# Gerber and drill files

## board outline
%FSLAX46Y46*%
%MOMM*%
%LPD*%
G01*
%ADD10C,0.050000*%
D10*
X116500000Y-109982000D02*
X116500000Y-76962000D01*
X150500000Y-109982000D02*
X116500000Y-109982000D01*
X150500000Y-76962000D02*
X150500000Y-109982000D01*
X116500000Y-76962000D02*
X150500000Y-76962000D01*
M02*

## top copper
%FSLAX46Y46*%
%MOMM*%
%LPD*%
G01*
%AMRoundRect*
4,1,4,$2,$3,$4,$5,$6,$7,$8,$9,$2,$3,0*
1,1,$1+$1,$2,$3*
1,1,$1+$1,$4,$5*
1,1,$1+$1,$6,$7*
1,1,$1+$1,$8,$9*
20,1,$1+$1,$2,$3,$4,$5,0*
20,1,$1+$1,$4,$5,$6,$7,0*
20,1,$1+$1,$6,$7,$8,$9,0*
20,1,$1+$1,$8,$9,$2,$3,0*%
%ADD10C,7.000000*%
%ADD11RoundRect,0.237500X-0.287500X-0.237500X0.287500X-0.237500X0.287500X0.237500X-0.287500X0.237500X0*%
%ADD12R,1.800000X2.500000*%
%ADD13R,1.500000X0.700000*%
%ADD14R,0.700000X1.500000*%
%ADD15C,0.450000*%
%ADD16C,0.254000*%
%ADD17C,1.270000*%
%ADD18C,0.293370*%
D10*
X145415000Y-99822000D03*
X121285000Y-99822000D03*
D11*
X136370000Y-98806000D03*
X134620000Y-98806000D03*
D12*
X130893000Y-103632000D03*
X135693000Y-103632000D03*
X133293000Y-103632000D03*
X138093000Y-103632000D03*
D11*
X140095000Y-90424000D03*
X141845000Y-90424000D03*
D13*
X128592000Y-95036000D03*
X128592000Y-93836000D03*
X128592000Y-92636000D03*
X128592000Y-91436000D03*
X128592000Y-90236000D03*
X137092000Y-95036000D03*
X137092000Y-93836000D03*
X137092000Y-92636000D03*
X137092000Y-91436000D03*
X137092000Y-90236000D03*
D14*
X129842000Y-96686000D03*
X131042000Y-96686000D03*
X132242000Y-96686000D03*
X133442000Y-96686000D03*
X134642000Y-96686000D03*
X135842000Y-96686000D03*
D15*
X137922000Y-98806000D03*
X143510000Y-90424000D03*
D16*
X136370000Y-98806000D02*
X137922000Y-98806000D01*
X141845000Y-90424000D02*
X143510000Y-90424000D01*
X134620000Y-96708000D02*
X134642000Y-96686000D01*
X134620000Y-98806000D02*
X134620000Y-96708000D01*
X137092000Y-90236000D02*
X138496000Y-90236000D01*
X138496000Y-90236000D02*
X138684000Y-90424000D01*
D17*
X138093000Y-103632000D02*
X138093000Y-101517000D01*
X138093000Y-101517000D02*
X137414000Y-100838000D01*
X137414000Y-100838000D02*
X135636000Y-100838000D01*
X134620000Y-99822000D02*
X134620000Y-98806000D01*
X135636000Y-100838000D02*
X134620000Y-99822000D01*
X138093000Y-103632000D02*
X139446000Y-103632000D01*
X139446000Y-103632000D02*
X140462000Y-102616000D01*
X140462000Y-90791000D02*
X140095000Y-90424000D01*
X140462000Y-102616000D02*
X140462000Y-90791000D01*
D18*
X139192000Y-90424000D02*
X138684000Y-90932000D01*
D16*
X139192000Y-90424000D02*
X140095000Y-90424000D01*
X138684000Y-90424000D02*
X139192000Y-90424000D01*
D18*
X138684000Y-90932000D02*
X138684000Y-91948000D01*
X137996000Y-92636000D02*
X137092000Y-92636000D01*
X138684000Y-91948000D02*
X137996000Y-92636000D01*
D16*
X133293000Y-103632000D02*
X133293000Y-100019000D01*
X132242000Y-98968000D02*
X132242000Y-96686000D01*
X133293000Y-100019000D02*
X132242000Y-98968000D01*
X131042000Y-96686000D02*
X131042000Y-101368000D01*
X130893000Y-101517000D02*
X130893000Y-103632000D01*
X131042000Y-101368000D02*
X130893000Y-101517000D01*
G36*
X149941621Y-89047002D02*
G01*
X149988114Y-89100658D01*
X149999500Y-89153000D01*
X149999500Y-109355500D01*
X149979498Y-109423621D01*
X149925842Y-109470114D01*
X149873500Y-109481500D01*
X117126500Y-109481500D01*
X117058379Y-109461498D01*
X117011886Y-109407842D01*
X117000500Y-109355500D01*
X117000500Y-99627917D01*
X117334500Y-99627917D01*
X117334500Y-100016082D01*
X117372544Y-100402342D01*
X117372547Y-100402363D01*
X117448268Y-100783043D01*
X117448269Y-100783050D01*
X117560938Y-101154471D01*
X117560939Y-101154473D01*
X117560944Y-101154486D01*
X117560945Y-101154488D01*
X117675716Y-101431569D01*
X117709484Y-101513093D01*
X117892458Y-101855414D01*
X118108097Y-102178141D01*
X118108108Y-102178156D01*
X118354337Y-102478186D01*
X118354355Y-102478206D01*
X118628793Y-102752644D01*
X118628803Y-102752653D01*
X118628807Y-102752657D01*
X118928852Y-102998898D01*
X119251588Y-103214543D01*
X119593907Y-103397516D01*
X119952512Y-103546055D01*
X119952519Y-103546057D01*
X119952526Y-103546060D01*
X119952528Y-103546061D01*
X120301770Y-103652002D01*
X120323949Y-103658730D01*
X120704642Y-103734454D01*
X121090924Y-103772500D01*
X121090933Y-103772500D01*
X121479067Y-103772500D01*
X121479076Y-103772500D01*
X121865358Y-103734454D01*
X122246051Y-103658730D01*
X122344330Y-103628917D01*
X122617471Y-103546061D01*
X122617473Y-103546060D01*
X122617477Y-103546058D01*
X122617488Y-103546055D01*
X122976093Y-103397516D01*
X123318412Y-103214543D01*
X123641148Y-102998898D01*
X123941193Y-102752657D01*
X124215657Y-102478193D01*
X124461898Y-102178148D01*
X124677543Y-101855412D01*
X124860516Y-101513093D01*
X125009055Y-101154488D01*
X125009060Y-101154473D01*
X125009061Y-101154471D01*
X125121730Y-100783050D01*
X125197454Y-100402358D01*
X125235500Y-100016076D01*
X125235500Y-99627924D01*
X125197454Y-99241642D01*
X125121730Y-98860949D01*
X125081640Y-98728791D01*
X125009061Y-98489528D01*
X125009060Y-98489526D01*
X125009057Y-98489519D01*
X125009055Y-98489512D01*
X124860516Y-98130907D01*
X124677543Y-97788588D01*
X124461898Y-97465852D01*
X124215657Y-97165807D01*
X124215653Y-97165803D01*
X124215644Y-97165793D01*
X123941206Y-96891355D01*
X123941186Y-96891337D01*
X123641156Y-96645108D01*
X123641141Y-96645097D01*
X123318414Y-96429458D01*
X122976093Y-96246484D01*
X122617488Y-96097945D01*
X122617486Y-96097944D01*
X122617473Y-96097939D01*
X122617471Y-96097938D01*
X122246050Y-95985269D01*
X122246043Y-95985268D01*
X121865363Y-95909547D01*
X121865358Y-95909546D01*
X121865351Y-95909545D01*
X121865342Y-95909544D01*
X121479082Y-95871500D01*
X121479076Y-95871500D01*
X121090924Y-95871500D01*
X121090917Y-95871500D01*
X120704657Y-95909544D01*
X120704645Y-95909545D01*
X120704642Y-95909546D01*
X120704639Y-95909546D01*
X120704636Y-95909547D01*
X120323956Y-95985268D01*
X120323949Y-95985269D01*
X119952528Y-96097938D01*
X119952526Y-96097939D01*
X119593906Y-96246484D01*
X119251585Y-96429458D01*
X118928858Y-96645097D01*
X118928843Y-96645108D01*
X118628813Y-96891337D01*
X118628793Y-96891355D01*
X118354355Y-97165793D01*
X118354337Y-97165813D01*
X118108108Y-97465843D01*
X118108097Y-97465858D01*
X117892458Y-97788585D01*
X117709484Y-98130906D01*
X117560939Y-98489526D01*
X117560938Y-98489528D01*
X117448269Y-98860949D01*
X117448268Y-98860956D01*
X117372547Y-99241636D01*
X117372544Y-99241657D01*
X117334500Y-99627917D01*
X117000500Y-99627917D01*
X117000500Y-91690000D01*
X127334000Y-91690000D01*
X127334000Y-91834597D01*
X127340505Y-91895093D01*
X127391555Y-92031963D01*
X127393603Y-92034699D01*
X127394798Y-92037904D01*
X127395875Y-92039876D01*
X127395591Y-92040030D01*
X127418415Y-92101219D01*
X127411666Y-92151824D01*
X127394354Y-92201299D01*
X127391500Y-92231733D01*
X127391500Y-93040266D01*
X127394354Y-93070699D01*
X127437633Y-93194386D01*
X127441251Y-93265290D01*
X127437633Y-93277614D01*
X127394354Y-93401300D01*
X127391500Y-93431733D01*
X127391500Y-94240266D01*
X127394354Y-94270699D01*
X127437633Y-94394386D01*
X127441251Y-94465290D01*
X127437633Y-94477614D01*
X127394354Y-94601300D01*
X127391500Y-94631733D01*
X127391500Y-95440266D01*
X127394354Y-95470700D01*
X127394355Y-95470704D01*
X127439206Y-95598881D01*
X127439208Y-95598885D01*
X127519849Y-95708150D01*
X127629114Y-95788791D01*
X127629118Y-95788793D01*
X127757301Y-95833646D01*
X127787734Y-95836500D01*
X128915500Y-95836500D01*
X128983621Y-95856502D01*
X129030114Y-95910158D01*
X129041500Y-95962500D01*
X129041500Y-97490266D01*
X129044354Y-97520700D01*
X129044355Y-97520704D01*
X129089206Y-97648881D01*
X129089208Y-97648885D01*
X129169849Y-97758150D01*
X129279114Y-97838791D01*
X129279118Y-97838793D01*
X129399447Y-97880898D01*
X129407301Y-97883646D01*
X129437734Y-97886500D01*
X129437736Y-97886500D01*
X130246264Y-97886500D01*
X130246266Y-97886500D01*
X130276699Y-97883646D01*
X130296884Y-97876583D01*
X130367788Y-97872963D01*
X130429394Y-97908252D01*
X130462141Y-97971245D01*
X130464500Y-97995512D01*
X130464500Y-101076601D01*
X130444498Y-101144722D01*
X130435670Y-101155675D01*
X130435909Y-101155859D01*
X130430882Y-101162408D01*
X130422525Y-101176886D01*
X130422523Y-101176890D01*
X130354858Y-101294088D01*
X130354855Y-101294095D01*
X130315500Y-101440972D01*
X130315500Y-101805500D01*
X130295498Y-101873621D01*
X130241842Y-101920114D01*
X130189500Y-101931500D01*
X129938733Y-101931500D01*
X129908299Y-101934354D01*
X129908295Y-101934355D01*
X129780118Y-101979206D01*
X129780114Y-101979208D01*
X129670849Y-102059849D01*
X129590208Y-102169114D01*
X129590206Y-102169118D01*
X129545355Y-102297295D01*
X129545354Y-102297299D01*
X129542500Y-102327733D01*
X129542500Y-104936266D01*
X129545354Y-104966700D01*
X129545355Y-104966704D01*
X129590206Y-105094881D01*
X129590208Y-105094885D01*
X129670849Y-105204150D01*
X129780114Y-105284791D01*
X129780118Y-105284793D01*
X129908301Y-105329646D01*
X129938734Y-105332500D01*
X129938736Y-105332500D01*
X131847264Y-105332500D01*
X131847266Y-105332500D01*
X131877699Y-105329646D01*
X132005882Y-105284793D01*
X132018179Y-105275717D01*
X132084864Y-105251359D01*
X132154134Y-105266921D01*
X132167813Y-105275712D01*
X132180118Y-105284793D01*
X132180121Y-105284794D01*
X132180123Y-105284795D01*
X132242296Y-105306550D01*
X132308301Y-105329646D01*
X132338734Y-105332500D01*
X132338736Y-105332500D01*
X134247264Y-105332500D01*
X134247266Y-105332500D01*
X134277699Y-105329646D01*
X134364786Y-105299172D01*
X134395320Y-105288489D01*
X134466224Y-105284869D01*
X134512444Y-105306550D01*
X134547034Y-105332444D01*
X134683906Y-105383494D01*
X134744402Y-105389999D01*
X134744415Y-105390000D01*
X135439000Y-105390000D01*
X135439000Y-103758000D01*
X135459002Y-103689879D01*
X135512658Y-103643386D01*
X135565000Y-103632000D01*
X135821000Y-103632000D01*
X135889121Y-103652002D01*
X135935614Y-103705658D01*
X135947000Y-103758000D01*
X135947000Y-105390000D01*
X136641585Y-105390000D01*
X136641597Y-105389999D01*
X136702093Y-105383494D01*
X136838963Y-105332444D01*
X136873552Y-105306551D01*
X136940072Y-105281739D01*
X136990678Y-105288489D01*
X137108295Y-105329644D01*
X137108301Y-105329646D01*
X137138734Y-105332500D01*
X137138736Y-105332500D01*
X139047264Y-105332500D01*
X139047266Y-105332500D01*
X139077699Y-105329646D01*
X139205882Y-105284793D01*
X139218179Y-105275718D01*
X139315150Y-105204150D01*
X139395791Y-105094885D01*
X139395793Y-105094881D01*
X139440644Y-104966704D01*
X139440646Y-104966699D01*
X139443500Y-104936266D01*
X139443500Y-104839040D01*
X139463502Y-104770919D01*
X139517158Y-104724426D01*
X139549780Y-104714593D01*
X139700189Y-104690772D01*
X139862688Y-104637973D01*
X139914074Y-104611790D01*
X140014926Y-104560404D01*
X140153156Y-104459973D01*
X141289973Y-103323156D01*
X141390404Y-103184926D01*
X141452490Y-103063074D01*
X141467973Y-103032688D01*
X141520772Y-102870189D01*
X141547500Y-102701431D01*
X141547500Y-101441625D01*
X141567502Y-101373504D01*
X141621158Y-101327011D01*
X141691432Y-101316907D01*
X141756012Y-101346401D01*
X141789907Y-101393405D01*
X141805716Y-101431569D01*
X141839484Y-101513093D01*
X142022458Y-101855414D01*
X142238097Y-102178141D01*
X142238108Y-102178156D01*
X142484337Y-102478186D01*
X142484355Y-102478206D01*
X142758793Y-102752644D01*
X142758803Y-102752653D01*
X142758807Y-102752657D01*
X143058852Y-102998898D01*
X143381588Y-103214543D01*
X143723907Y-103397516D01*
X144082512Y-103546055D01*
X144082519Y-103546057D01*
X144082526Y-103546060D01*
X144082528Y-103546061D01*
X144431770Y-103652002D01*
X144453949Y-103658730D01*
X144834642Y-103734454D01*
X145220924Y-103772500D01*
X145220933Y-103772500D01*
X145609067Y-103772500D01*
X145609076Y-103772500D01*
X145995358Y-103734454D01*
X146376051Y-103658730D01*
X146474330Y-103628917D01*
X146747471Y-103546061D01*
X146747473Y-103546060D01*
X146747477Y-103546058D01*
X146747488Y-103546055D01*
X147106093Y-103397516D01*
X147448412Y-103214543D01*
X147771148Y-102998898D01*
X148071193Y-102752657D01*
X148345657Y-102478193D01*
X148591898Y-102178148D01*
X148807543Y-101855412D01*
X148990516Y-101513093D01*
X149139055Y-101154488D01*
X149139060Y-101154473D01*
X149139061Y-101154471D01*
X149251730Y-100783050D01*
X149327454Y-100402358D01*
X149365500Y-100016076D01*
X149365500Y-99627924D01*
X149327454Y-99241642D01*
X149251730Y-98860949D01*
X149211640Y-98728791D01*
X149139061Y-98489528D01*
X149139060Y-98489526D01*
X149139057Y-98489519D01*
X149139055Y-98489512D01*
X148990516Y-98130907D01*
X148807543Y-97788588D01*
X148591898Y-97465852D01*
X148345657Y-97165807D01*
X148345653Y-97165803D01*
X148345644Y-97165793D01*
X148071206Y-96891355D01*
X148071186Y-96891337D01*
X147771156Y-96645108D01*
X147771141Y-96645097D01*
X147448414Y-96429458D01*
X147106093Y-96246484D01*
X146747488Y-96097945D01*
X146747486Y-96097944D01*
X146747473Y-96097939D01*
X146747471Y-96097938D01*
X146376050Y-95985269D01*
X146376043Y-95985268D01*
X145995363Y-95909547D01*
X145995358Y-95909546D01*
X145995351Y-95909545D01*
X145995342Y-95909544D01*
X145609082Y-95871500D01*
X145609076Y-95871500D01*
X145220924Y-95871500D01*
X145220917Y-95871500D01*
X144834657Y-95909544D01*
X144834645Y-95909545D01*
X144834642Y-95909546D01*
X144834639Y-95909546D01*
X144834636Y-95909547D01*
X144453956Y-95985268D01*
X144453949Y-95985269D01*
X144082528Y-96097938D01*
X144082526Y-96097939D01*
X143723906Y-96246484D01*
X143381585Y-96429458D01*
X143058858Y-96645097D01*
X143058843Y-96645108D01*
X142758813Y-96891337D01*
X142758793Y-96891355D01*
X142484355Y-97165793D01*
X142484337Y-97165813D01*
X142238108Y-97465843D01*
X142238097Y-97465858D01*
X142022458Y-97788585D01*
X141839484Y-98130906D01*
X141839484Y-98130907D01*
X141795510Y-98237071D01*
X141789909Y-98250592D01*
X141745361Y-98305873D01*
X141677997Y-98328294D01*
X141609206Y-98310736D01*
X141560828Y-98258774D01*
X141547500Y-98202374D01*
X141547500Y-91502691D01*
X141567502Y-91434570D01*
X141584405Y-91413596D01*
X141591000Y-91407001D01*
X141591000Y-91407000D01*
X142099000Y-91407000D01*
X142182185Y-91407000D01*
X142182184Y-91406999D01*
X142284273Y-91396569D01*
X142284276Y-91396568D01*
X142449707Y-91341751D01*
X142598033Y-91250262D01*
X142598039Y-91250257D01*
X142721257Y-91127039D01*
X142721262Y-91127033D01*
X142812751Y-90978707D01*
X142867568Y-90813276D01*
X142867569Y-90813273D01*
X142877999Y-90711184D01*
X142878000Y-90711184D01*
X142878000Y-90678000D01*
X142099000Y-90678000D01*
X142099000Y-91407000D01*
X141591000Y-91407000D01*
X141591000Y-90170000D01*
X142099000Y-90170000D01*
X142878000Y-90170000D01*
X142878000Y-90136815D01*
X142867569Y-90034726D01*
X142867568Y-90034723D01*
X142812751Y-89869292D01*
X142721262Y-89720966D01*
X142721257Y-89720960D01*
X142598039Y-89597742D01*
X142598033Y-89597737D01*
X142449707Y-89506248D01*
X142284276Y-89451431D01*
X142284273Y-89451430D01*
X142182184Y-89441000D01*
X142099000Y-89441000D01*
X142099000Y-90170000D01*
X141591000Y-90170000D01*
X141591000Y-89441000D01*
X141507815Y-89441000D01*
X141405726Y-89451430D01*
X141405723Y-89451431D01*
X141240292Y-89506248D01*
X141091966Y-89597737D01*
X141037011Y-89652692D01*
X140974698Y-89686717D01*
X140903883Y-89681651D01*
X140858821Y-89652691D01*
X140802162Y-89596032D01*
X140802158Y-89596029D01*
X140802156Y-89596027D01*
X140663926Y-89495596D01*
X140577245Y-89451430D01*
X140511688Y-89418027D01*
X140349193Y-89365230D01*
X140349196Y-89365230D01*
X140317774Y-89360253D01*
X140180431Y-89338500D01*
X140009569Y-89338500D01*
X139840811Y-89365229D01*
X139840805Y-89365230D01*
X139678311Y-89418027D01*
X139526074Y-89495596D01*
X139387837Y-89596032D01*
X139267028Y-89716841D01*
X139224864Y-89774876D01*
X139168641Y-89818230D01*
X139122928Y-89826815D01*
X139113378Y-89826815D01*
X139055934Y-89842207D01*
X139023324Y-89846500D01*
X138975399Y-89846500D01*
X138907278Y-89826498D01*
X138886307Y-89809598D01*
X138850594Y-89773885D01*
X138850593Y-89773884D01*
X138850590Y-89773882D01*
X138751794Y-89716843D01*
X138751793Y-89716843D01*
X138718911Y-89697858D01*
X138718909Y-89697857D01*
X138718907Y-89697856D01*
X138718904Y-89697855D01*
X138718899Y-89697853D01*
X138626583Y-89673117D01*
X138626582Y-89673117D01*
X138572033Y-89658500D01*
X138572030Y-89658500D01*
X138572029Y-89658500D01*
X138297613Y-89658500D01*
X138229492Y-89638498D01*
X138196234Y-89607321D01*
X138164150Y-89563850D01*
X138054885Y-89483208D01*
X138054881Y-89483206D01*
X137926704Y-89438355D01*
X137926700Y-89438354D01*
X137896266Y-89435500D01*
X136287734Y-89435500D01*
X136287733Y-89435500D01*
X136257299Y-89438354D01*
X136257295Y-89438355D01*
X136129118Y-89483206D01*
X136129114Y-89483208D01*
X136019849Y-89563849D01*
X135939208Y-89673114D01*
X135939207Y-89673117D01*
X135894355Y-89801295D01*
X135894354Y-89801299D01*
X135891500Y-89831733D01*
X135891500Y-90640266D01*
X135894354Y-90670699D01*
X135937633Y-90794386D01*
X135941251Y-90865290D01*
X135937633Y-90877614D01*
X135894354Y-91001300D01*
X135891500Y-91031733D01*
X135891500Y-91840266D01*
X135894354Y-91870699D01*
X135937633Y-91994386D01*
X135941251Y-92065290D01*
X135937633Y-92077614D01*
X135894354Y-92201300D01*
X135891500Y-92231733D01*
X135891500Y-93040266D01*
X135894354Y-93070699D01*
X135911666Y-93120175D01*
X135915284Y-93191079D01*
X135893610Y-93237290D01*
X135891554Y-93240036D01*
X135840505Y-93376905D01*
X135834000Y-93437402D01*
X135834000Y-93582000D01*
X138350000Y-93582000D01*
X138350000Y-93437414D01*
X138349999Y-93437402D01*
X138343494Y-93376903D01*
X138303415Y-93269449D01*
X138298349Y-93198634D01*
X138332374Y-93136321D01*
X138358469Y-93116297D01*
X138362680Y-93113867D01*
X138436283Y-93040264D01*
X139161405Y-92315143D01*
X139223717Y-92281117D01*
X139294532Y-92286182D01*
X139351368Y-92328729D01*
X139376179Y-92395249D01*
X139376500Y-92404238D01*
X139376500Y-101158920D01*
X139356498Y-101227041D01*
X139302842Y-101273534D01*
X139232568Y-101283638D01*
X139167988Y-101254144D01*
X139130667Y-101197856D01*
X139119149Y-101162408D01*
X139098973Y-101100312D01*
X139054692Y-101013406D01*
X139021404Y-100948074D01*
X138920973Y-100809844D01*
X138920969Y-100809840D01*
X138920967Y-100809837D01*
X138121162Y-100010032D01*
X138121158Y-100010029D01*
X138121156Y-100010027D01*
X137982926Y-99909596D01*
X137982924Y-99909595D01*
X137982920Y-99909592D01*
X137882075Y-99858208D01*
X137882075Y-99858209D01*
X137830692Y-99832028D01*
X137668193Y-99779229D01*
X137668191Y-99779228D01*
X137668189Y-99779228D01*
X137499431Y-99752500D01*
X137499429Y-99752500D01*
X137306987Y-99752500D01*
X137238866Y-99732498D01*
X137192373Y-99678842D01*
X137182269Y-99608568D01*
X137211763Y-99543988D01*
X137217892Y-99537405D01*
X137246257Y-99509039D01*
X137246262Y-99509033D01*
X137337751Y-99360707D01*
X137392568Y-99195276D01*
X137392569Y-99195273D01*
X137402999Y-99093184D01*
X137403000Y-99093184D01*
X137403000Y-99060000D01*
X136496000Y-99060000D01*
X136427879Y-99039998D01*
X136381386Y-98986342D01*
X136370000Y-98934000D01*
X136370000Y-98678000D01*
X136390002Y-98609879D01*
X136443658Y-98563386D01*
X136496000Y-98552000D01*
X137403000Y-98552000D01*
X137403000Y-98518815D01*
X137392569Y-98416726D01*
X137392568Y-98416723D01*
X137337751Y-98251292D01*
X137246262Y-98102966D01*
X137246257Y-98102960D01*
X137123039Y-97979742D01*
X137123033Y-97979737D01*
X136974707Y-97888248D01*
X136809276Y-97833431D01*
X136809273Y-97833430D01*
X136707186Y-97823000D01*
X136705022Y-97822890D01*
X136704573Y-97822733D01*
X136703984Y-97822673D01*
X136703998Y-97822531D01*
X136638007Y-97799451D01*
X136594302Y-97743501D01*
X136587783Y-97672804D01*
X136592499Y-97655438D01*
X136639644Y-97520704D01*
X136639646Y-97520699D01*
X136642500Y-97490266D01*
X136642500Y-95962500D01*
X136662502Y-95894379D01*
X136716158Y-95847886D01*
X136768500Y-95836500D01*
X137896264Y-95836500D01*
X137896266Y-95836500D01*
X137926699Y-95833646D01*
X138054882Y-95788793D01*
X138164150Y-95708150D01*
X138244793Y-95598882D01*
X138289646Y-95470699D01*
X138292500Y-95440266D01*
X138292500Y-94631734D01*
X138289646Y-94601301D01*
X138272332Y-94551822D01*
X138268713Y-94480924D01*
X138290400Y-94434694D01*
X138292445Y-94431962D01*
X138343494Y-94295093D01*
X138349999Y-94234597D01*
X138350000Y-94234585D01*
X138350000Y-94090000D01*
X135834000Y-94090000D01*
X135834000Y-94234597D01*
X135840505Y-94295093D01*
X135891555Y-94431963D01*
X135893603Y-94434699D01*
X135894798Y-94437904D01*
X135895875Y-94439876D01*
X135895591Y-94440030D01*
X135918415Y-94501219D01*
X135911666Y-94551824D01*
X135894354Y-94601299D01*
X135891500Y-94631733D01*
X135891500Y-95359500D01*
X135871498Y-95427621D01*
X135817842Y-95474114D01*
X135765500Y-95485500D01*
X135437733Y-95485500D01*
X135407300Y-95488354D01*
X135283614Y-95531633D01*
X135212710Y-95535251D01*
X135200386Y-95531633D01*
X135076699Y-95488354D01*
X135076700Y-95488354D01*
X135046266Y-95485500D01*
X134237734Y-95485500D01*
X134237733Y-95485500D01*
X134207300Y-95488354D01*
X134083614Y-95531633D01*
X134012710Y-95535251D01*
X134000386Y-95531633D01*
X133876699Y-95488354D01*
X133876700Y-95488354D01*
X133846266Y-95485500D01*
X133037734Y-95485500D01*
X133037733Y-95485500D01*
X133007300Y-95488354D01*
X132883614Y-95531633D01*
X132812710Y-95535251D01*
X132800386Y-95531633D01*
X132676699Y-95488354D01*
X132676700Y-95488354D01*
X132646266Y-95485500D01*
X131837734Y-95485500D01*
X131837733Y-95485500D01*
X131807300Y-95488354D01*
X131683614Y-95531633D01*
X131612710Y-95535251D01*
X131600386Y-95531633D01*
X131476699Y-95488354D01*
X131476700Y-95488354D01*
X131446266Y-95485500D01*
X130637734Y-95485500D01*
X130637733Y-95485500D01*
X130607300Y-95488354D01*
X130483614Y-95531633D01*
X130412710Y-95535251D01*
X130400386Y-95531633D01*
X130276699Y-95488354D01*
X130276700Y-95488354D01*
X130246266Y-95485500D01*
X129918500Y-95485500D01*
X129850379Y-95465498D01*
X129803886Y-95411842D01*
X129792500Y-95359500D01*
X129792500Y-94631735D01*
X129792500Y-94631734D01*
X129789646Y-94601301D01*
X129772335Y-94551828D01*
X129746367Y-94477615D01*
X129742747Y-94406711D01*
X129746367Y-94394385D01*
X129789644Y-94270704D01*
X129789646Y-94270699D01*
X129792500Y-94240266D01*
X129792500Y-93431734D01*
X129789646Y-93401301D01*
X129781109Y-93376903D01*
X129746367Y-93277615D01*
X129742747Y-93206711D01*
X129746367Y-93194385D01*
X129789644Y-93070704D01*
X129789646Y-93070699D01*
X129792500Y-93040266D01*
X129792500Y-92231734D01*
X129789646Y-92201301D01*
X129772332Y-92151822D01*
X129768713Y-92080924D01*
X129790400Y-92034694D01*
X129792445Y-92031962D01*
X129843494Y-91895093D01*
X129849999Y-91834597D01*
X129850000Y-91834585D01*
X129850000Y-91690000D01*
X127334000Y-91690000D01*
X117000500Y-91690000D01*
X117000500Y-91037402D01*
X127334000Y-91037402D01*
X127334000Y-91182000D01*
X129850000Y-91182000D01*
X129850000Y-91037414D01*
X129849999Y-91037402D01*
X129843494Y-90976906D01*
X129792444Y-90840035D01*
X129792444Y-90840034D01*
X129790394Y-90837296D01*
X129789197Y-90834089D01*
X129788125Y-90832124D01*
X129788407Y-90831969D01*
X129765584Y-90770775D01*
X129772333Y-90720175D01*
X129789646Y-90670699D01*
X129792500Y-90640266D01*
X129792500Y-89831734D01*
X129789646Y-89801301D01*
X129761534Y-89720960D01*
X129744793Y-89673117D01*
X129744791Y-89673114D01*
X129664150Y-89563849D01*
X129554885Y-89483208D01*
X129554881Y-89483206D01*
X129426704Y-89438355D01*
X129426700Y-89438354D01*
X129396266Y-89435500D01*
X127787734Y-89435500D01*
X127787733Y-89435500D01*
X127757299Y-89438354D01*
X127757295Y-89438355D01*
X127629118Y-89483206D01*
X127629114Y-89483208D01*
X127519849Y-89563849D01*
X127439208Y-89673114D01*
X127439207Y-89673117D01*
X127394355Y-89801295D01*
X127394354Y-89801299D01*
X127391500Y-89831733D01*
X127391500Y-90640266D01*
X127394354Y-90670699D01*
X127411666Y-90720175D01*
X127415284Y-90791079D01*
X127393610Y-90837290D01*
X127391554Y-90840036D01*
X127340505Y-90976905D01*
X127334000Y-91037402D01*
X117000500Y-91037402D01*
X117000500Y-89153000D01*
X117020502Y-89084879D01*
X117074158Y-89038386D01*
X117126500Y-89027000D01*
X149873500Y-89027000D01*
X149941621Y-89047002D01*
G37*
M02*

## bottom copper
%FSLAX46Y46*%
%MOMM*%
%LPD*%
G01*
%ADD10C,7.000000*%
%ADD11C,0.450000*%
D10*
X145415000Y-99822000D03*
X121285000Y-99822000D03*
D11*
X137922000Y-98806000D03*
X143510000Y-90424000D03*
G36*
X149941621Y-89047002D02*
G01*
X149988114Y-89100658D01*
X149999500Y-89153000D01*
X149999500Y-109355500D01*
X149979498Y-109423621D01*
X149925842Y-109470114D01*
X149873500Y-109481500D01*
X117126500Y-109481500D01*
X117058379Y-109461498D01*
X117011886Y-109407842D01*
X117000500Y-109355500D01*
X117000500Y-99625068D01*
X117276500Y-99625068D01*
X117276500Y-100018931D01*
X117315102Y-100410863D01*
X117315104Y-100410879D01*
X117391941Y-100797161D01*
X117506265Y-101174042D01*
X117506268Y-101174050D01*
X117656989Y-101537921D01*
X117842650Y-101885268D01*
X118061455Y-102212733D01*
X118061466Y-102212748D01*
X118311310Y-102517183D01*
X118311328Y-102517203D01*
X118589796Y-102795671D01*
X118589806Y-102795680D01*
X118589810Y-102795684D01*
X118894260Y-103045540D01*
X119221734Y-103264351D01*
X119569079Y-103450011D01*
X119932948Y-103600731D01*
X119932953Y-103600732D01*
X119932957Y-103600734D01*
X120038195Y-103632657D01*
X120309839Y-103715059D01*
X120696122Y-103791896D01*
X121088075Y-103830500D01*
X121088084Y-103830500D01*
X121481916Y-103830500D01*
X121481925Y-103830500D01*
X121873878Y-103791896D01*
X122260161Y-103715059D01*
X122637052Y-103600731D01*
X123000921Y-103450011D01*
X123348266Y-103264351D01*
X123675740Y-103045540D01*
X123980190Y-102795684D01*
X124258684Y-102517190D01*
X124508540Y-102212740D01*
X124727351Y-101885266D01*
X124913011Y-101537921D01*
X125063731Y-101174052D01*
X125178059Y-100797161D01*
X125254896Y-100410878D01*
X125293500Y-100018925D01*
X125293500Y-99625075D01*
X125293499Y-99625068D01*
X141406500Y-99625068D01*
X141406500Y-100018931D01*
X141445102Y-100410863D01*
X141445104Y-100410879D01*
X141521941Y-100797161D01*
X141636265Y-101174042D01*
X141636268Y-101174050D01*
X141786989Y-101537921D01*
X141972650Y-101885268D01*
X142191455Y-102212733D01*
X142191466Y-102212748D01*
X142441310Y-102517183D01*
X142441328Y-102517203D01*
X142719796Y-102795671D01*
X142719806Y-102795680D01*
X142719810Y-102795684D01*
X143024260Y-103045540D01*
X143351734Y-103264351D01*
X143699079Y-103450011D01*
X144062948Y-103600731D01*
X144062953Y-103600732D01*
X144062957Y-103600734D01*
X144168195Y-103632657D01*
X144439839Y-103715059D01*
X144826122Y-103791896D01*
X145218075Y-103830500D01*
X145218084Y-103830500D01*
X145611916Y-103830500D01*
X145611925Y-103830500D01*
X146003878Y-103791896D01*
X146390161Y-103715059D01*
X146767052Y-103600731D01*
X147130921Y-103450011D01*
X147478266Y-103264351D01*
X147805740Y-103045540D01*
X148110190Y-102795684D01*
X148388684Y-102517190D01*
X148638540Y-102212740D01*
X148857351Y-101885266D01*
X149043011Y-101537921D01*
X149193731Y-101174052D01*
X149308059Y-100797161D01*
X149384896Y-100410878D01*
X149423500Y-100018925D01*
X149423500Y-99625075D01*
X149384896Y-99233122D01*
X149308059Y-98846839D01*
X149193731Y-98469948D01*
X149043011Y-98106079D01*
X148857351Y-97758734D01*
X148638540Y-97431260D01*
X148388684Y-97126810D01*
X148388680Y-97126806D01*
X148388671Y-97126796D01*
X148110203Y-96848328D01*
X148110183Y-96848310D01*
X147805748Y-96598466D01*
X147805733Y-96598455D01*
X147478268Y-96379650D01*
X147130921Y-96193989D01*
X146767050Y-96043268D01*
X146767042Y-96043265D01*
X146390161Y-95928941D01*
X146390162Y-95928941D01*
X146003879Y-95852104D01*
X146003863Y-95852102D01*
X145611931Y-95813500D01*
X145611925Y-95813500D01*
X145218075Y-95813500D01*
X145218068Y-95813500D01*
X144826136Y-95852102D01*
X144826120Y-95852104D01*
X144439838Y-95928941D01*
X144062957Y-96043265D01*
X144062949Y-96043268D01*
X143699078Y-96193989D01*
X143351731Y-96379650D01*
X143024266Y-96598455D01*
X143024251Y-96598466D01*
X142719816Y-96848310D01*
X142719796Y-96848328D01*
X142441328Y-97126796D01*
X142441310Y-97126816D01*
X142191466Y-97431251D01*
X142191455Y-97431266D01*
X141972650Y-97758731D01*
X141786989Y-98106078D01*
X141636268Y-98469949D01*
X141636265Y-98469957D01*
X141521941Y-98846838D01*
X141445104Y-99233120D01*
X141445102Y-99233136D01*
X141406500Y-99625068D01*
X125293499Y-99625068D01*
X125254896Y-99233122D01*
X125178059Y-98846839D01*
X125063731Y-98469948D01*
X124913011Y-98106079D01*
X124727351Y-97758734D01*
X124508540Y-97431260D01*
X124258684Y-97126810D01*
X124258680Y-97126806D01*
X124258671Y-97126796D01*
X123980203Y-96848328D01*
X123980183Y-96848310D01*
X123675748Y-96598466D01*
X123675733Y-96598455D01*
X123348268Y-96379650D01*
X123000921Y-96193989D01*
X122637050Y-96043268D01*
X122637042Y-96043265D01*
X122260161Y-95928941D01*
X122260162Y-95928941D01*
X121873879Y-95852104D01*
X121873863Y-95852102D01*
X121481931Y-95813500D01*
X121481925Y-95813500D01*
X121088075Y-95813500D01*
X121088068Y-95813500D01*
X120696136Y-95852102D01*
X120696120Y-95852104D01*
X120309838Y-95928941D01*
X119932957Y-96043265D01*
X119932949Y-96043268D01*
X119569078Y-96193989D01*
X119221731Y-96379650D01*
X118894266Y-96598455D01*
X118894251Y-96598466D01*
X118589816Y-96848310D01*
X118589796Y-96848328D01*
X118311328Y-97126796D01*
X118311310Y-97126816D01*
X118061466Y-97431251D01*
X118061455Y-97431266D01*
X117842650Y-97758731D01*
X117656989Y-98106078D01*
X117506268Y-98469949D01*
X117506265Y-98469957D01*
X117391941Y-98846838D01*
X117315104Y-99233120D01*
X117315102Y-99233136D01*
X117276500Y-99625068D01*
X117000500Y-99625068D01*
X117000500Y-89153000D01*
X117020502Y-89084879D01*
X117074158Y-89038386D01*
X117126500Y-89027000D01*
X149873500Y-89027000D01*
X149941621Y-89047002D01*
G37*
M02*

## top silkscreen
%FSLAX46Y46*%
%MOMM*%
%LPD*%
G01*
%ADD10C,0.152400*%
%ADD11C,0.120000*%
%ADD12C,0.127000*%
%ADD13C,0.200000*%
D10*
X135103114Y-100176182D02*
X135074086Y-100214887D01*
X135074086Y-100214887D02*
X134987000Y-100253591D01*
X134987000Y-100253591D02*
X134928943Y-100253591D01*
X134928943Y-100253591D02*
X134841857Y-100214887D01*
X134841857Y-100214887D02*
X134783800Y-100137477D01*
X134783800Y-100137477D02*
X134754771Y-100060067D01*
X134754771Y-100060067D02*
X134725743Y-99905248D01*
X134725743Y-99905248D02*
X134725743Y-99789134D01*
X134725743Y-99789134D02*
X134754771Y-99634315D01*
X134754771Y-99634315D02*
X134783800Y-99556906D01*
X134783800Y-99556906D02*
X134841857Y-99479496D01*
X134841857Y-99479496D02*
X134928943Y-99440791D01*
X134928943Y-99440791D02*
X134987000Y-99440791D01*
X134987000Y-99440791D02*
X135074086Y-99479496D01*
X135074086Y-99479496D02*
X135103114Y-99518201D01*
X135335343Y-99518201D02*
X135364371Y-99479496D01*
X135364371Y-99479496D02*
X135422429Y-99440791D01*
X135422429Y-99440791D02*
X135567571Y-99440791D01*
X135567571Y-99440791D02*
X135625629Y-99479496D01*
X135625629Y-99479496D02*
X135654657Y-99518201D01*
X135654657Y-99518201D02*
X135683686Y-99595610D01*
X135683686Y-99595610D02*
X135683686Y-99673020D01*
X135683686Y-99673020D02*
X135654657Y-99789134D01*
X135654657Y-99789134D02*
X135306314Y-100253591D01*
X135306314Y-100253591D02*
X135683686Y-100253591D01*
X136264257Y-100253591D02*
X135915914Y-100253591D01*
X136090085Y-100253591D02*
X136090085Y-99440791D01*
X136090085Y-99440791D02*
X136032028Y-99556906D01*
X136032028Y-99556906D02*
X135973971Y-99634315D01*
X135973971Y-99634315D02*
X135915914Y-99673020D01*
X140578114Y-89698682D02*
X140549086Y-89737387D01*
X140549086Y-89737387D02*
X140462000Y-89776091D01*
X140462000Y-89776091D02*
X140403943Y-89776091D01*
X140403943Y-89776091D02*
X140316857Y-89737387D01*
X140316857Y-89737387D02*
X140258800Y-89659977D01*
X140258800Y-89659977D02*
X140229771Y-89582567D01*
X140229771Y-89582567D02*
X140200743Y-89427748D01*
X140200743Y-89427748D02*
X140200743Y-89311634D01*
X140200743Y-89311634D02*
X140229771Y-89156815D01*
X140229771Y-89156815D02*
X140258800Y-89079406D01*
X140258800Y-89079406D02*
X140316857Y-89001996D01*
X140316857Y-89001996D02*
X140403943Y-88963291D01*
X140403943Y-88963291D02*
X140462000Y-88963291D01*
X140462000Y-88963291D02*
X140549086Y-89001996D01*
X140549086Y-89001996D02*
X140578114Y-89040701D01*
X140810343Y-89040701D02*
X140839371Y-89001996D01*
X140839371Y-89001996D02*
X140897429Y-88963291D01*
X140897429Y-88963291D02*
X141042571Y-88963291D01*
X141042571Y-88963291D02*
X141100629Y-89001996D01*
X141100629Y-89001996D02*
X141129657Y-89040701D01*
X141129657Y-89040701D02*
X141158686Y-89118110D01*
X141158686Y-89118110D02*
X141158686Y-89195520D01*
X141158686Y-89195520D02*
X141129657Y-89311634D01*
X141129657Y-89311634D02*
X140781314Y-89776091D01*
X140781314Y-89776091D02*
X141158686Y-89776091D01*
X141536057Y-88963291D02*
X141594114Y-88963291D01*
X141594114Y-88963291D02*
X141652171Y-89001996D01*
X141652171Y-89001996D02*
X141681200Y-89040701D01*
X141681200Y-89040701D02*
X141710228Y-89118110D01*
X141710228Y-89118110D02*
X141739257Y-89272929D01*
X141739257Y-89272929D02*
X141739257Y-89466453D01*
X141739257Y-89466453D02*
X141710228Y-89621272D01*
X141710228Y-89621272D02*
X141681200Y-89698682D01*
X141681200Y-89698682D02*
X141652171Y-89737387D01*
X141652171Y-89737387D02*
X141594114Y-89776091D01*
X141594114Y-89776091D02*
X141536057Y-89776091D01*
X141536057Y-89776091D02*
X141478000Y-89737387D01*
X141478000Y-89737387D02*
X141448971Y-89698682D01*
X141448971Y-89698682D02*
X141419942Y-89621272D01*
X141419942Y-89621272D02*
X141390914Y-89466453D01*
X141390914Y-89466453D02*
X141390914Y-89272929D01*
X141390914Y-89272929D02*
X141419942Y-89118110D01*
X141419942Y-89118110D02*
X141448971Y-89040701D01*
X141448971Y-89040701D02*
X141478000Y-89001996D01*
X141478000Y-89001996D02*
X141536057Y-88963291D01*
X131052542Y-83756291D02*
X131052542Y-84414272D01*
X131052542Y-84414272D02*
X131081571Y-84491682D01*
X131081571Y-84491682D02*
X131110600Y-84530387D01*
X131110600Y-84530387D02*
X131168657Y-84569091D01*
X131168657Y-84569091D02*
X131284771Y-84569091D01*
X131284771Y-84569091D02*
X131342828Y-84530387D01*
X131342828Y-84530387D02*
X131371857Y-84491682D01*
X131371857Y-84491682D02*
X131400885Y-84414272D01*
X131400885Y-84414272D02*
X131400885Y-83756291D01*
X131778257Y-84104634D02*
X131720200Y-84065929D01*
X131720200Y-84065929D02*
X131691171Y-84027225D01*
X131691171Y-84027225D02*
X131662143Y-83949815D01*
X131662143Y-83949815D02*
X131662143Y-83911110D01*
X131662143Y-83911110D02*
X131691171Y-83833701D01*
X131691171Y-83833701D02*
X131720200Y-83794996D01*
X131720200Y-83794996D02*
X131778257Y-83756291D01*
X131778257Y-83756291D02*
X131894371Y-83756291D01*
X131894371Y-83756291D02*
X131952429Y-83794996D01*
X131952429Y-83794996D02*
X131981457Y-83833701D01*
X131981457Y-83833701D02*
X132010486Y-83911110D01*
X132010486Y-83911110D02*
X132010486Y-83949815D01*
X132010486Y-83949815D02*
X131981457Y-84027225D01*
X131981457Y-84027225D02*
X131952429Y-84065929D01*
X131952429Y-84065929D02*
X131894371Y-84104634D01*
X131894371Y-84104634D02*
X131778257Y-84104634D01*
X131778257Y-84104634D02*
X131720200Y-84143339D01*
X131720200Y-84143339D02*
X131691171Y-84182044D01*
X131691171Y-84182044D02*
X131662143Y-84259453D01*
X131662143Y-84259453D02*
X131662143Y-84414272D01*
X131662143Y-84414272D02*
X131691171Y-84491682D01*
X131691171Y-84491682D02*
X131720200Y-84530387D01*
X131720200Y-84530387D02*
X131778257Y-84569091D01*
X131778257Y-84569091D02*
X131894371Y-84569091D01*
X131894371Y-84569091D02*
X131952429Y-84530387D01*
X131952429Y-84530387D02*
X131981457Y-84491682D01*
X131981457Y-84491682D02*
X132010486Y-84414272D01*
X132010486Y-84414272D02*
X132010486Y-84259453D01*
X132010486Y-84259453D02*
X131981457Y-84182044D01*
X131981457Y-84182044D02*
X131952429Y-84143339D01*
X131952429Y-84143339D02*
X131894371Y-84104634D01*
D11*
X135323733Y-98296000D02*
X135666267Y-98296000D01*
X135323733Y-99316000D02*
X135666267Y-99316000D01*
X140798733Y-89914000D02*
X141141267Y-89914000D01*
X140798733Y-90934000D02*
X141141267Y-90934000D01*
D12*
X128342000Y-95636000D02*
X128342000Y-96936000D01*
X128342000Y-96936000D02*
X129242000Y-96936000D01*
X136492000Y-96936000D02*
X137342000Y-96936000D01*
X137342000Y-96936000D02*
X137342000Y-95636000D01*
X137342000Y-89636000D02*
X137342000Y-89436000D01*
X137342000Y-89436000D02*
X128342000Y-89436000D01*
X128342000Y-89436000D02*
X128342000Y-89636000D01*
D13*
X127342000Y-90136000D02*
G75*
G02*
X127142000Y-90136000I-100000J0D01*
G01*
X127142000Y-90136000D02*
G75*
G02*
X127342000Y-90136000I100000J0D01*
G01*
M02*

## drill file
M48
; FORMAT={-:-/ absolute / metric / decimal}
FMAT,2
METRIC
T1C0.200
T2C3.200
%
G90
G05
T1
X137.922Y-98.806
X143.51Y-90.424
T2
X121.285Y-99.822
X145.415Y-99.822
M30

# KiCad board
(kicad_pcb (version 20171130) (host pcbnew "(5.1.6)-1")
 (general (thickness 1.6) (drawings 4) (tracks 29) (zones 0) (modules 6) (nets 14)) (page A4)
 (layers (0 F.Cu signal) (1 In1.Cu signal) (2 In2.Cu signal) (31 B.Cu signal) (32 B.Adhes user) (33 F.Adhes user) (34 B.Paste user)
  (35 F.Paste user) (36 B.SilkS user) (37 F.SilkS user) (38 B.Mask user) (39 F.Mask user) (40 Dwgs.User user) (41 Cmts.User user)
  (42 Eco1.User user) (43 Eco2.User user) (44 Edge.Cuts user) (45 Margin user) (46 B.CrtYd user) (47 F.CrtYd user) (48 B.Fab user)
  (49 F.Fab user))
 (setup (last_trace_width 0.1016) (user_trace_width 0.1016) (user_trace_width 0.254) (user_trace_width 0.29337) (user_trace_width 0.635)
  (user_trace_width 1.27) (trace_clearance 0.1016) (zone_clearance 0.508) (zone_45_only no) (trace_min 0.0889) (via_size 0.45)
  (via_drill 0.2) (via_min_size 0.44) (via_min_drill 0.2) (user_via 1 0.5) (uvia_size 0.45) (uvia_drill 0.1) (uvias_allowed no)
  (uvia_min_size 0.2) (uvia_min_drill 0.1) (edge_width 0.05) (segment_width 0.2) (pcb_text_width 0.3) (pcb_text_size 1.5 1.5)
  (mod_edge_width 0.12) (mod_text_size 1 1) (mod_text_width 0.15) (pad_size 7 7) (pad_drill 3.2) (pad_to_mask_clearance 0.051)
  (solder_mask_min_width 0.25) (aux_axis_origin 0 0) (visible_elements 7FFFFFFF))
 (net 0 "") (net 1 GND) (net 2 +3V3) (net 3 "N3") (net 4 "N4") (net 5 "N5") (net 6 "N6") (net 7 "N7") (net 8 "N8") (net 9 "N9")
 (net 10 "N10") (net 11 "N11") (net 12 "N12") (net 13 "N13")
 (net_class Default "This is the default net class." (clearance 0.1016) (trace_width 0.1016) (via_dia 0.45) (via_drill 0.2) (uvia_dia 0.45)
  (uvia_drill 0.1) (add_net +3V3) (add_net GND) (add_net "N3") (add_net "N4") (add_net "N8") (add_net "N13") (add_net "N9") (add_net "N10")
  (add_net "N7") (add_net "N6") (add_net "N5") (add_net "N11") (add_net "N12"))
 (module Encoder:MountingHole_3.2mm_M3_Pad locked (layer F.Cu) (at 145.415 99.822)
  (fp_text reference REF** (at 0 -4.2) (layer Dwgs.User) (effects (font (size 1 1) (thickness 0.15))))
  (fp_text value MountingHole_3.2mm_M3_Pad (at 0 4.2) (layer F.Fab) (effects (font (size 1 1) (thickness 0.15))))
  (pad 1 thru_hole circle (at 0 0) (size 7 7) (drill 3.2) (layers *.Cu *.Mask)))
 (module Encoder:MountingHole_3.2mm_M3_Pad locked (layer F.Cu) (at 121.285 99.822)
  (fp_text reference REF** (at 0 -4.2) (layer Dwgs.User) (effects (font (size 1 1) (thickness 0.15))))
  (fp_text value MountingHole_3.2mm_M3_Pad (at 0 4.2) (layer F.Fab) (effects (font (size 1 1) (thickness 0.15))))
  (pad 1 thru_hole circle (at 0 0) (size 7 7) (drill 3.2) (layers *.Cu *.Mask)))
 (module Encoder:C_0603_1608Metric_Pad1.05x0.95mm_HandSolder (layer F.Cu) (at 135.495 98.806)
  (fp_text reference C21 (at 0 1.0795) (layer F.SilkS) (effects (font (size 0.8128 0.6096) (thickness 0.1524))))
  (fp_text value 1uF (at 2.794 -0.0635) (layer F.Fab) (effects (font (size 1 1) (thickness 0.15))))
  (fp_line (start -0.171267 -0.51) (end 0.171267 -0.51) (layer F.SilkS) (width 0.12))
  (fp_line (start -0.171267 0.51) (end 0.171267 0.51) (layer F.SilkS) (width 0.12))
  (pad 2 smd roundrect (at 0.875 0) (size 1.05 0.95) (layers F.Cu F.Paste F.Mask) (roundrect_rratio 0.25) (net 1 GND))
  (pad 1 smd roundrect (at -0.875 0) (size 1.05 0.95) (layers F.Cu F.Paste F.Mask) (roundrect_rratio 0.25) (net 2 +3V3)))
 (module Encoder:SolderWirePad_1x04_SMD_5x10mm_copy (layer F.Cu) (at 134.493 103.632)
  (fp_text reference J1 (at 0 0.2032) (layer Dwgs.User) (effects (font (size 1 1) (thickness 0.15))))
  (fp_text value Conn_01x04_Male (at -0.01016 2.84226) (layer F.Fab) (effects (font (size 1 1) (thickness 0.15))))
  (pad 1 smd rect (at -3.6 0) (size 1.8 2.5) (layers F.Cu F.Paste F.Mask) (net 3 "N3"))
  (pad 3 smd rect (at 1.2 0) (size 1.8 2.5) (layers F.Cu F.Paste F.Mask) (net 1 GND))
  (pad 2 smd rect (at -1.2 0) (size 1.8 2.5) (layers F.Cu F.Paste F.Mask) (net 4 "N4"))
  (pad 4 smd rect (at 3.6 0) (size 1.8 2.5) (layers F.Cu F.Paste F.Mask) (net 2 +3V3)))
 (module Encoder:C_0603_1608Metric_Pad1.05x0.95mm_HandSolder (layer F.Cu) (at 140.97 90.424)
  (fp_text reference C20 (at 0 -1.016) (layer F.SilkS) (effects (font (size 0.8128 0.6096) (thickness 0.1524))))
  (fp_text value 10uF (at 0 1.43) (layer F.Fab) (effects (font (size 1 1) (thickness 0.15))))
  (fp_line (start -0.171267 -0.51) (end 0.171267 -0.51) (layer F.SilkS) (width 0.12))
  (fp_line (start -0.171267 0.51) (end 0.171267 0.51) (layer F.SilkS) (width 0.12))
  (pad 1 smd roundrect (at -0.875 0) (size 1.05 0.95) (layers F.Cu F.Paste F.Mask) (roundrect_rratio 0.25) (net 2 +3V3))
  (pad 2 smd roundrect (at 0.875 0) (size 1.05 0.95) (layers F.Cu F.Paste F.Mask) (roundrect_rratio 0.25) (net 1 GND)))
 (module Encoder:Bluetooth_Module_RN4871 (layer F.Cu) (at 132.842 91.186)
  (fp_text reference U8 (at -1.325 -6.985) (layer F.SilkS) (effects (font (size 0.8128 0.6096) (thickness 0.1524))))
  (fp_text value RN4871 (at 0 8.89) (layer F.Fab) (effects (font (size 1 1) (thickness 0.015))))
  (fp_line (start -4.5 4.45) (end -4.5 5.75) (layer F.SilkS) (width 0.127))
  (fp_line (start -4.5 5.75) (end -3.6 5.75) (layer F.SilkS) (width 0.127))
  (fp_line (start 3.65 5.75) (end 4.5 5.75) (layer F.SilkS) (width 0.127))
  (fp_line (start 4.5 5.75) (end 4.5 4.45) (layer F.SilkS) (width 0.127))
  (fp_line (start 4.5 -1.55) (end 4.5 -1.75) (layer F.SilkS) (width 0.127))
  (fp_line (start 4.5 -1.75) (end -4.5 -1.75) (layer F.SilkS) (width 0.127))
  (fp_line (start -4.5 -1.75) (end -4.5 -1.55) (layer F.SilkS) (width 0.127))
  (fp_circle (center -5.6 -1.05) (end -5.5 -1.05) (layer F.SilkS) (width 0.2))
  (pad 5 smd rect (at -4.25 3.85) (size 1.5 0.7) (layers F.Cu F.Paste F.Mask) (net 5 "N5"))
  (pad 4 smd rect (at -4.25 2.65) (size 1.5 0.7) (layers F.Cu F.Paste F.Mask) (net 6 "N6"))
  (pad 3 smd rect (at -4.25 1.45) (size 1.5 0.7) (layers F.Cu F.Paste F.Mask) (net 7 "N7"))
  (pad 2 smd rect (at -4.25 0.25) (size 1.5 0.7) (layers F.Cu F.Paste F.Mask) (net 1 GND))
  (pad 1 smd rect (at -4.25 -0.95) (size 1.5 0.7) (layers F.Cu F.Paste F.Mask) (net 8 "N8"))
  (pad 12 smd rect (at 4.25 3.85) (size 1.5 0.7) (layers F.Cu F.Paste F.Mask) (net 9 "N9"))
  (pad 13 smd rect (at 4.25 2.65) (size 1.5 0.7) (layers F.Cu F.Paste F.Mask) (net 1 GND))
  (pad 14 smd rect (at 4.25 1.45) (size 1.5 0.7) (layers F.Cu F.Paste F.Mask) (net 2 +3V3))
  (pad 15 smd rect (at 4.25 0.25) (size 1.5 0.7) (layers F.Cu F.Paste F.Mask) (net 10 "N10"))
  (pad 16 smd rect (at 4.25 -0.95) (size 1.5 0.7) (layers F.Cu F.Paste F.Mask) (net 2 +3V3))
  (pad 6 smd rect (at -3 5.5) (size 0.7 1.5) (layers F.Cu F.Paste F.Mask) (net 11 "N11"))
  (pad 7 smd rect (at -1.8 5.5) (size 0.7 1.5) (layers F.Cu F.Paste F.Mask) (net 3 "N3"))
  (pad 8 smd rect (at -0.6 5.5) (size 0.7 1.5) (layers F.Cu F.Paste F.Mask) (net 4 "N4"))
  (pad 9 smd rect (at 0.6 5.5) (size 0.7 1.5) (layers F.Cu F.Paste F.Mask) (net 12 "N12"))
  (pad 10 smd rect (at 1.8 5.5) (size 0.7 1.5) (layers F.Cu F.Paste F.Mask) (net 2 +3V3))
  (pad 11 smd rect (at 3 5.5) (size 0.7 1.5) (layers F.Cu F.Paste F.Mask) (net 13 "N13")))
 (gr_line (start 116.5 109.982) (end 116.5 76.962) (layer Edge.Cuts) (width 0.05))
 (gr_line (start 150.5 109.982) (end 116.5 109.982) (layer Edge.Cuts) (width 0.05))
 (gr_line (start 150.5 76.962) (end 150.5 109.982) (layer Edge.Cuts) (width 0.05))
 (gr_line (start 116.5 76.962) (end 150.5 76.962) (layer Edge.Cuts) (width 0.05))
 (segment (start 136.37 98.806) (end 137.922 98.806) (width 0.254) (layer F.Cu) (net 1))
 (via (at 137.922 98.806) (size 0.45) (drill 0.2) (layers F.Cu B.Cu) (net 1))
 (segment (start 141.845 90.424) (end 143.51 90.424) (width 0.254) (layer F.Cu) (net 1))
 (via (at 143.51 90.424) (size 0.45) (drill 0.2) (layers F.Cu B.Cu) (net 1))
 (segment (start 134.62 96.708) (end 134.642 96.686) (width 0.254) (layer F.Cu) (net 2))
 (segment (start 134.62 98.806) (end 134.62 96.708) (width 0.254) (layer F.Cu) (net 2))
 (segment (start 137.092 90.236) (end 138.496 90.236) (width 0.254) (layer F.Cu) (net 2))
 (segment (start 138.496 90.236) (end 138.684 90.424) (width 0.254) (layer F.Cu) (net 2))
 (segment (start 138.093 103.632) (end 138.093 101.517) (width 1.27) (layer F.Cu) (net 2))
 (segment (start 138.093 101.517) (end 137.414 100.838) (width 1.27) (layer F.Cu) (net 2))
 (segment (start 137.414 100.838) (end 135.636 100.838) (width 1.27) (layer F.Cu) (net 2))
 (segment (start 134.62 99.822) (end 134.62 98.806) (width 1.27) (layer F.Cu) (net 2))
 (segment (start 135.636 100.838) (end 134.62 99.822) (width 1.27) (layer F.Cu) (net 2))
 (segment (start 138.093 103.632) (end 139.446 103.632) (width 1.27) (layer F.Cu) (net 2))
 (segment (start 139.446 103.632) (end 140.462 102.616) (width 1.27) (layer F.Cu) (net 2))
 (segment (start 140.462 90.791) (end 140.095 90.424) (width 1.27) (layer F.Cu) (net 2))
 (segment (start 140.462 102.616) (end 140.462 90.791) (width 1.27) (layer F.Cu) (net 2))
 (segment (start 139.192 90.424) (end 138.684 90.932) (width 0.29337) (layer F.Cu) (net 2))
 (segment (start 139.192 90.424) (end 140.095 90.424) (width 0.254) (layer F.Cu) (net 2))
 (segment (start 138.684 90.424) (end 139.192 90.424) (width 0.254) (layer F.Cu) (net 2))
 (segment (start 138.684 90.932) (end 138.684 91.948) (width 0.29337) (layer F.Cu) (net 2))
 (segment (start 137.996 92.636) (end 137.092 92.636) (width 0.29337) (layer F.Cu) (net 2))
 (segment (start 138.684 91.948) (end 137.996 92.636) (width 0.29337) (layer F.Cu) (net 2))
 (segment (start 133.293 103.632) (end 133.293 100.019) (width 0.254) (layer F.Cu) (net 4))
 (segment (start 132.242 98.968) (end 132.242 96.686) (width 0.254) (layer F.Cu) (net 4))
 (segment (start 133.293 100.019) (end 132.242 98.968) (width 0.254) (layer F.Cu) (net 4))
 (segment (start 131.042 96.686) (end 131.042 101.368) (width 0.254) (layer F.Cu) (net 3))
 (segment (start 130.893 101.517) (end 130.893 103.632) (width 0.254) (layer F.Cu) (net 3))
 (segment (start 131.042 101.368) (end 130.893 101.517) (width 0.254) (layer F.Cu) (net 3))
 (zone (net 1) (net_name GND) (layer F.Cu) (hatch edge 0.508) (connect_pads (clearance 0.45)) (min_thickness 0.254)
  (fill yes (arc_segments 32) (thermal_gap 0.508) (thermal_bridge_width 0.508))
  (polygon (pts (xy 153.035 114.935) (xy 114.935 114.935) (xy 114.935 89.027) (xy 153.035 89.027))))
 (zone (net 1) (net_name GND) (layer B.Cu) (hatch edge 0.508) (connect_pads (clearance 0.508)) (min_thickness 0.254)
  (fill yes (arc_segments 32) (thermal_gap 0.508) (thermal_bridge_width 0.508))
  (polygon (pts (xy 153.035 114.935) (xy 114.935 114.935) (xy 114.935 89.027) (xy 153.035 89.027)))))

